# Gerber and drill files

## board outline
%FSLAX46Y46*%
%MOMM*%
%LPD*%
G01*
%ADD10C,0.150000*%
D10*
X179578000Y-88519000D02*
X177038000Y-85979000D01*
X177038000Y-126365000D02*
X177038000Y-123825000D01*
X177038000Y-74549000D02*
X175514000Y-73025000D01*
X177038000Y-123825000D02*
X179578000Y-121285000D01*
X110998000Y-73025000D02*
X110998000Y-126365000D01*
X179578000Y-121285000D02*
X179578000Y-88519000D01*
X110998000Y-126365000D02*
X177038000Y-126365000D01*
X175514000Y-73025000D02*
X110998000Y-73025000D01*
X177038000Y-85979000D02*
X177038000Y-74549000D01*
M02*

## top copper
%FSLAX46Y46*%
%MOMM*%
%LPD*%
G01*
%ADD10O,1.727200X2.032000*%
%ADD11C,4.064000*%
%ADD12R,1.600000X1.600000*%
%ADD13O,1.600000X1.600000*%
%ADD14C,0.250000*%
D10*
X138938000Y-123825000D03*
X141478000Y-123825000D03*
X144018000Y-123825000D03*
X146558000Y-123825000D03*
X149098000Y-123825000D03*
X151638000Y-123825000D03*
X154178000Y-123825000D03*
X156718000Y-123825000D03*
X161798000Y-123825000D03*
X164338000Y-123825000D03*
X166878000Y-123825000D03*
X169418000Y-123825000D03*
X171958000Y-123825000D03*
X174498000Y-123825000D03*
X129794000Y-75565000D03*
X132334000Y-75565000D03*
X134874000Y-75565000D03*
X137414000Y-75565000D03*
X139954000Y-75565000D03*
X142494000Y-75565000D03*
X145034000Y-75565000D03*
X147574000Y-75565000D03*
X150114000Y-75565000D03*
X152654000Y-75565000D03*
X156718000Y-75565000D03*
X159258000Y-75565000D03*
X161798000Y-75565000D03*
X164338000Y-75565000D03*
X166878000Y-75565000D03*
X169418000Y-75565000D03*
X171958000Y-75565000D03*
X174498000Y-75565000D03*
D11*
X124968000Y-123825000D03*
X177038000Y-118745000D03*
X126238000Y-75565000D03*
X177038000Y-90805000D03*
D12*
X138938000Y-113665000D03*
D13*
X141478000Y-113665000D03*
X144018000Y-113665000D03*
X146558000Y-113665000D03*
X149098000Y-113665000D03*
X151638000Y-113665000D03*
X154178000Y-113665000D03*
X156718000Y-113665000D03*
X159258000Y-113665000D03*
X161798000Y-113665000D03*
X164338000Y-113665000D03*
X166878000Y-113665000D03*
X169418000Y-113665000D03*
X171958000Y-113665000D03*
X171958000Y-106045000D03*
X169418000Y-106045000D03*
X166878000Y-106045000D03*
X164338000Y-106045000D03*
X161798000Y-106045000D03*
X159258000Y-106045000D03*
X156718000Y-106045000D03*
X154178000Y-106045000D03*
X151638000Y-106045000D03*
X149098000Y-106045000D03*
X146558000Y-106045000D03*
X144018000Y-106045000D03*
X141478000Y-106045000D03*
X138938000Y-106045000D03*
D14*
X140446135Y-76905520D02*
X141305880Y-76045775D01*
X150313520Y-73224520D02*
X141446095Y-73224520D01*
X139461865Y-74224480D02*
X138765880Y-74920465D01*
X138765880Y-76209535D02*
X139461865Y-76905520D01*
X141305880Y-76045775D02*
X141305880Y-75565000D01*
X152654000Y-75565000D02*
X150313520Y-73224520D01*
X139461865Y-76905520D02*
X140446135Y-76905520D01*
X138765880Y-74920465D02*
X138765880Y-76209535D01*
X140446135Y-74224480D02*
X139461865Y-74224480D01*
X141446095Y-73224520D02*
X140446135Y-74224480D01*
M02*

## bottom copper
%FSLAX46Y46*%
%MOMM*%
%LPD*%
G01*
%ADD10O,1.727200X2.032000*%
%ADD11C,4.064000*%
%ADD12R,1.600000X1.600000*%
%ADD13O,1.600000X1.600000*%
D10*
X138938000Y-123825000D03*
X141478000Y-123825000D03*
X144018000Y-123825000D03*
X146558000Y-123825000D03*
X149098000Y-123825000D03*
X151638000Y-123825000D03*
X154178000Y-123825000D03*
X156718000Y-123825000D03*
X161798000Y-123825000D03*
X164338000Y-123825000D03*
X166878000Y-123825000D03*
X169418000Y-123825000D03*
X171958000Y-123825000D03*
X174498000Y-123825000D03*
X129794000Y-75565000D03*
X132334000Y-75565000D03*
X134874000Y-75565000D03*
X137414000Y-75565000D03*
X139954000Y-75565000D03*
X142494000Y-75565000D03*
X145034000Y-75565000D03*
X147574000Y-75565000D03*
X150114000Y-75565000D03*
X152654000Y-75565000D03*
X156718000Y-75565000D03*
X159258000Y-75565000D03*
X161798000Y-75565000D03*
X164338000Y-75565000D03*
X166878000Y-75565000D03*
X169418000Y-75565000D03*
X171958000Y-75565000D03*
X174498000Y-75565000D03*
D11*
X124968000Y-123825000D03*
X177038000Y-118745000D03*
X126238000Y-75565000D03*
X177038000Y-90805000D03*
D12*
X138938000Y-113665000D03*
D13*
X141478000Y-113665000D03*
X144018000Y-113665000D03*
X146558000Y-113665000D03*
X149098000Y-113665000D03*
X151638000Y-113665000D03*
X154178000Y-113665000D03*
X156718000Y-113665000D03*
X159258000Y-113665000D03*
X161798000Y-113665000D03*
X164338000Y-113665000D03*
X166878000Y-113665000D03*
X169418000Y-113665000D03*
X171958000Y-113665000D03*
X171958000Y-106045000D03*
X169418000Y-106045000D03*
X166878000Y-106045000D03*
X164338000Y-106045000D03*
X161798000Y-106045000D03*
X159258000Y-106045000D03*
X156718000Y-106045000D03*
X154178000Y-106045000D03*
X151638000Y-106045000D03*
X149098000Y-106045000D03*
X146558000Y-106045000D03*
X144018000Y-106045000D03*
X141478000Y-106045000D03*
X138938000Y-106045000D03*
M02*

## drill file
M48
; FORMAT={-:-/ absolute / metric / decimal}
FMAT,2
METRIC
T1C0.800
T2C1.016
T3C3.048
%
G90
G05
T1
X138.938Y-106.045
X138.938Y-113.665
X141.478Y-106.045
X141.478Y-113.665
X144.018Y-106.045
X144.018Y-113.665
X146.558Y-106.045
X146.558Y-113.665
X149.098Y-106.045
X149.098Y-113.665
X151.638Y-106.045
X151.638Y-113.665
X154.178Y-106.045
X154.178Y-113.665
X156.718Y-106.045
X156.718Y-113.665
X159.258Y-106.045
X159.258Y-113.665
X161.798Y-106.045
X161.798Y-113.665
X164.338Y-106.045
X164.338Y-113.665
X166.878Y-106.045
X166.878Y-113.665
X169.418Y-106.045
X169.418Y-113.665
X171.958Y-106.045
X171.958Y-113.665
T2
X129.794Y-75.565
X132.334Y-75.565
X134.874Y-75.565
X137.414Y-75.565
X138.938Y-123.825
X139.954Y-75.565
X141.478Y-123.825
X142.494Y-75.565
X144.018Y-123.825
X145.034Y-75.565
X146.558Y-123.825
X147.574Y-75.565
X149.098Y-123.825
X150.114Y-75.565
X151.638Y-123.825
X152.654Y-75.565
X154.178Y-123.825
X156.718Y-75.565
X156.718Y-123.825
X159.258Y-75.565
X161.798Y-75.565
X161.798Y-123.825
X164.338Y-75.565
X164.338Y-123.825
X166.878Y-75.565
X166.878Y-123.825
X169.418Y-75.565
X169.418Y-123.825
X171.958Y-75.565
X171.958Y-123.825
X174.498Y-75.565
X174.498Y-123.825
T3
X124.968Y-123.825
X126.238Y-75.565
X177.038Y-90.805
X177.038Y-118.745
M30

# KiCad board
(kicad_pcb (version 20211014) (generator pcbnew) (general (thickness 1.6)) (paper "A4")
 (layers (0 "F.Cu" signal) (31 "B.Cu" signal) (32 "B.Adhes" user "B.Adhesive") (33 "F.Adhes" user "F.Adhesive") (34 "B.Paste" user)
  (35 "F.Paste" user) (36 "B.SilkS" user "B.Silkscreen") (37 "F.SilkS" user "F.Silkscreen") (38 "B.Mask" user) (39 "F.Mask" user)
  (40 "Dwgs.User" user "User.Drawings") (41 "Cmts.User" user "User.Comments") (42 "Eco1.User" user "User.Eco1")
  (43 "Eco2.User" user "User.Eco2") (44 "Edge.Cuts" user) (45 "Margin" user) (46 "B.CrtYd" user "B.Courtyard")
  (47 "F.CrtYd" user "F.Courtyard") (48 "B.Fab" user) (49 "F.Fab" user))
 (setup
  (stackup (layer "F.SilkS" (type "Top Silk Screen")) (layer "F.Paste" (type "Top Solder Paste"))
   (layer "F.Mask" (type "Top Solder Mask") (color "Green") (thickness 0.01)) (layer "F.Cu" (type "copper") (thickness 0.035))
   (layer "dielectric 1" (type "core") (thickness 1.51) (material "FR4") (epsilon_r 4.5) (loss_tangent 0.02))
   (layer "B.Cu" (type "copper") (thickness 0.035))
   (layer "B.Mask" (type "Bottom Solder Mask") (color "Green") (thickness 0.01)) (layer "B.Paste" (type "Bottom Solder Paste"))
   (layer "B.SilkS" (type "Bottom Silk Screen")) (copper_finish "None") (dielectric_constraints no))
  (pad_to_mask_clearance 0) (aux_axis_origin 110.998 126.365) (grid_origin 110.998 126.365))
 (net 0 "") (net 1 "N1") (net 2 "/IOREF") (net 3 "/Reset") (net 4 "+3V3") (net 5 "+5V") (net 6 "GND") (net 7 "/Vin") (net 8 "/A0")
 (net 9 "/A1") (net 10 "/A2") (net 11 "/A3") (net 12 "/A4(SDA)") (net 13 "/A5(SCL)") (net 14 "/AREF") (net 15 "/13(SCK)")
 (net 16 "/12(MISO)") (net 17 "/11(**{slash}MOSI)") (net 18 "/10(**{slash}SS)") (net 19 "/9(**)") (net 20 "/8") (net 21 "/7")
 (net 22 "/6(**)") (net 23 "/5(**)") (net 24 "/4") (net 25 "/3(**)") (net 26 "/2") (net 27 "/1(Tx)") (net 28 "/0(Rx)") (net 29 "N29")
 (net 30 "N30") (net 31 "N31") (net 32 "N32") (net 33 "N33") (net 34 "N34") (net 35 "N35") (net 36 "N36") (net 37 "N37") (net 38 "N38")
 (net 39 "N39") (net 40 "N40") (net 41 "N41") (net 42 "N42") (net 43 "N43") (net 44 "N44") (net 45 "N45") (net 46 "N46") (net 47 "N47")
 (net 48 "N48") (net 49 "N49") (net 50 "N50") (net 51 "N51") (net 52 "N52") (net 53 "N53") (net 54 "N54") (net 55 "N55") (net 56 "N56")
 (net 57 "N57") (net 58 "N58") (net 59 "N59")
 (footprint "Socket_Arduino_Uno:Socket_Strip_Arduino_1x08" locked (layer "F.Cu") (at 138.938 123.825)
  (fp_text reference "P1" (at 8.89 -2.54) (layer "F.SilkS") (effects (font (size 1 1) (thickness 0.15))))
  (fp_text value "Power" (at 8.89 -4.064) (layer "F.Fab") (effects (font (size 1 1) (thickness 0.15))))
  (pad "1" thru_hole oval locked (at 0 0) (size 1.7272 2.032) (drill 1.016) (layers *.Cu *.Mask "F.SilkS") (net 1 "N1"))
  (pad "2" thru_hole oval locked (at 2.54 0) (size 1.7272 2.032) (drill 1.016) (layers *.Cu *.Mask "F.SilkS") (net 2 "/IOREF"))
  (pad "3" thru_hole oval locked (at 5.08 0) (size 1.7272 2.032) (drill 1.016) (layers *.Cu *.Mask "F.SilkS") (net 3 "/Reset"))
  (pad "4" thru_hole oval locked (at 7.62 0) (size 1.7272 2.032) (drill 1.016) (layers *.Cu *.Mask "F.SilkS") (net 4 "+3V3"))
  (pad "5" thru_hole oval locked (at 10.16 0) (size 1.7272 2.032) (drill 1.016) (layers *.Cu *.Mask "F.SilkS") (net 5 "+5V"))
  (pad "6" thru_hole oval locked (at 12.7 0) (size 1.7272 2.032) (drill 1.016) (layers *.Cu *.Mask "F.SilkS") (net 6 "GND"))
  (pad "7" thru_hole oval locked (at 15.24 0) (size 1.7272 2.032) (drill 1.016) (layers *.Cu *.Mask "F.SilkS") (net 6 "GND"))
  (pad "8" thru_hole oval locked (at 17.78 0) (size 1.7272 2.032) (drill 1.016) (layers *.Cu *.Mask "F.SilkS") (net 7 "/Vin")))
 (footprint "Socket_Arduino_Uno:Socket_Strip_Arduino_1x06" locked (layer "F.Cu") (at 161.798 123.825)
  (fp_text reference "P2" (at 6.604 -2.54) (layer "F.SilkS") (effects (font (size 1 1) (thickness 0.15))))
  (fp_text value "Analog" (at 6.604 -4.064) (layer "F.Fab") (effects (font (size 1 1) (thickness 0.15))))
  (pad "1" thru_hole oval locked (at 0 0) (size 1.7272 2.032) (drill 1.016) (layers *.Cu *.Mask "F.SilkS") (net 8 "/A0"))
  (pad "2" thru_hole oval locked (at 2.54 0) (size 1.7272 2.032) (drill 1.016) (layers *.Cu *.Mask "F.SilkS") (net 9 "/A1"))
  (pad "3" thru_hole oval locked (at 5.08 0) (size 1.7272 2.032) (drill 1.016) (layers *.Cu *.Mask "F.SilkS") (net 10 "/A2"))
  (pad "4" thru_hole oval locked (at 7.62 0) (size 1.7272 2.032) (drill 1.016) (layers *.Cu *.Mask "F.SilkS") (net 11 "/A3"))
  (pad "5" thru_hole oval locked (at 10.16 0) (size 1.7272 2.032) (drill 1.016) (layers *.Cu *.Mask "F.SilkS") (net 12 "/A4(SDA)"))
  (pad "6" thru_hole oval locked (at 12.7 0) (size 1.7272 2.032) (drill 1.016) (layers *.Cu *.Mask "F.SilkS") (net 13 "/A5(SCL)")))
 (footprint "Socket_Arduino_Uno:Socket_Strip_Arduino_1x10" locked (layer "F.Cu") (at 129.794 75.565)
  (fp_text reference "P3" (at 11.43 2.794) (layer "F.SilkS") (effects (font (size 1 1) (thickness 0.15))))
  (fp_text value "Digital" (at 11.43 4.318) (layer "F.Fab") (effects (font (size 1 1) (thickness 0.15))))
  (pad "1" thru_hole oval locked (at 0 0) (size 1.7272 2.032) (drill 1.016) (layers *.Cu *.Mask "F.SilkS") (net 13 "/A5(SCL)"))
  (pad "2" thru_hole oval locked (at 2.54 0) (size 1.7272 2.032) (drill 1.016) (layers *.Cu *.Mask "F.SilkS") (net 12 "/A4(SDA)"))
  (pad "3" thru_hole oval locked (at 5.08 0) (size 1.7272 2.032) (drill 1.016) (layers *.Cu *.Mask "F.SilkS") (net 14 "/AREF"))
  (pad "4" thru_hole oval locked (at 7.62 0) (size 1.7272 2.032) (drill 1.016) (layers *.Cu *.Mask "F.SilkS") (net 6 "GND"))
  (pad "5" thru_hole oval locked (at 10.16 0) (size 1.7272 2.032) (drill 1.016) (layers *.Cu *.Mask "F.SilkS") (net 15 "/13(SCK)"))
  (pad "6" thru_hole oval locked (at 12.7 0) (size 1.7272 2.032) (drill 1.016) (layers *.Cu *.Mask "F.SilkS") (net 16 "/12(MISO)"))
  (pad "7" thru_hole oval locked (at 15.24 0) (size 1.7272 2.032) (drill 1.016) (layers *.Cu *.Mask "F.SilkS") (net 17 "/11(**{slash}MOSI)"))
  (pad "8" thru_hole oval locked (at 17.78 0) (size 1.7272 2.032) (drill 1.016) (layers *.Cu *.Mask "F.SilkS") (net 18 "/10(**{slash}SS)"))
  (pad "9" thru_hole oval locked (at 20.32 0) (size 1.7272 2.032) (drill 1.016) (layers *.Cu *.Mask "F.SilkS") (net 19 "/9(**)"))
  (pad "10" thru_hole oval locked (at 22.86 0) (size 1.7272 2.032) (drill 1.016) (layers *.Cu *.Mask "F.SilkS") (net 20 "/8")))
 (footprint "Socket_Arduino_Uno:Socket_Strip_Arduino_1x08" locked (layer "F.Cu") (at 156.718 75.565)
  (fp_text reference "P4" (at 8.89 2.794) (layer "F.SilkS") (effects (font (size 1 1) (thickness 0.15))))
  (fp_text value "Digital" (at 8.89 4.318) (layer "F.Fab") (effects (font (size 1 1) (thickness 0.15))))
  (pad "1" thru_hole oval locked (at 0 0) (size 1.7272 2.032) (drill 1.016) (layers *.Cu *.Mask "F.SilkS") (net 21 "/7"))
  (pad "2" thru_hole oval locked (at 2.54 0) (size 1.7272 2.032) (drill 1.016) (layers *.Cu *.Mask "F.SilkS") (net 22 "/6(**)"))
  (pad "3" thru_hole oval locked (at 5.08 0) (size 1.7272 2.032) (drill 1.016) (layers *.Cu *.Mask "F.SilkS") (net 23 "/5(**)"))
  (pad "4" thru_hole oval locked (at 7.62 0) (size 1.7272 2.032) (drill 1.016) (layers *.Cu *.Mask "F.SilkS") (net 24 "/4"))
  (pad "5" thru_hole oval locked (at 10.16 0) (size 1.7272 2.032) (drill 1.016) (layers *.Cu *.Mask "F.SilkS") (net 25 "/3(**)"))
  (pad "6" thru_hole oval locked (at 12.7 0) (size 1.7272 2.032) (drill 1.016) (layers *.Cu *.Mask "F.SilkS") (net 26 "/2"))
  (pad "7" thru_hole oval locked (at 15.24 0) (size 1.7272 2.032) (drill 1.016) (layers *.Cu *.Mask "F.SilkS") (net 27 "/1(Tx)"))
  (pad "8" thru_hole oval locked (at 17.78 0) (size 1.7272 2.032) (drill 1.016) (layers *.Cu *.Mask "F.SilkS") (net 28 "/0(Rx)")))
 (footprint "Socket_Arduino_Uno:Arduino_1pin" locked (layer "F.Cu") (at 124.968 123.825)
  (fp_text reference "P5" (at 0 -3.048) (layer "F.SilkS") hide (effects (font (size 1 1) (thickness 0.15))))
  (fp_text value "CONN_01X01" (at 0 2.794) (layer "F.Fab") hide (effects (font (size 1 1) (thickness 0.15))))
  (pad "1" thru_hole circle locked (at 0 0) (size 4.064 4.064) (drill 3.048) (layers *.Cu *.Mask "F.SilkS") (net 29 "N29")))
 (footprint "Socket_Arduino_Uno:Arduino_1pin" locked (layer "F.Cu") (at 177.038 118.745)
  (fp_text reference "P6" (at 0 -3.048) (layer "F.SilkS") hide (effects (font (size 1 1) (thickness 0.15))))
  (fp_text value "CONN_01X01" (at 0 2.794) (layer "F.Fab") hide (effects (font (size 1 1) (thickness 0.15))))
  (pad "1" thru_hole circle locked (at 0 0) (size 4.064 4.064) (drill 3.048) (layers *.Cu *.Mask "F.SilkS") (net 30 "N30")))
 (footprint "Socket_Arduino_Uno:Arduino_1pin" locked (layer "F.Cu") (at 126.238 75.565)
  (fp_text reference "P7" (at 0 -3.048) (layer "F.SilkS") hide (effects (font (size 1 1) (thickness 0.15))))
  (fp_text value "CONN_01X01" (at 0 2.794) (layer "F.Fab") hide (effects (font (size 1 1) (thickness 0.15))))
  (pad "1" thru_hole circle locked (at 0 0) (size 4.064 4.064) (drill 3.048) (layers *.Cu *.Mask "F.SilkS") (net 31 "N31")))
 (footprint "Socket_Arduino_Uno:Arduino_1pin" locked (layer "F.Cu") (at 177.038 90.805)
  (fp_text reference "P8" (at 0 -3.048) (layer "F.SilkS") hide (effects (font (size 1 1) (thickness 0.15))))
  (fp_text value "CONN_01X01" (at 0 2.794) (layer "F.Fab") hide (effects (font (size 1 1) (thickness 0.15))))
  (pad "1" thru_hole circle locked (at 0 0) (size 4.064 4.064) (drill 3.048) (layers *.Cu *.Mask "F.SilkS") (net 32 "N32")))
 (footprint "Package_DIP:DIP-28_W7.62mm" (layer "F.Cu") (at 138.938 113.665 90)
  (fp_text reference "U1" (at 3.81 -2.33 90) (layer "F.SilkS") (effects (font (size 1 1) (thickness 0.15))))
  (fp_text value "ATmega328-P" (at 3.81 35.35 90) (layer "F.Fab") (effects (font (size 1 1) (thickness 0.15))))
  (pad "1" thru_hole rect (at 0 0 90) (size 1.6 1.6) (drill 0.8) (layers *.Cu *.Mask) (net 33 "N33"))
  (pad "2" thru_hole oval (at 0 2.54 90) (size 1.6 1.6) (drill 0.8) (layers *.Cu *.Mask) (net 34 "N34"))
  (pad "3" thru_hole oval (at 0 5.08 90) (size 1.6 1.6) (drill 0.8) (layers *.Cu *.Mask) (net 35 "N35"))
  (pad "4" thru_hole oval (at 0 7.62 90) (size 1.6 1.6) (drill 0.8) (layers *.Cu *.Mask) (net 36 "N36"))
  (pad "5" thru_hole oval (at 0 10.16 90) (size 1.6 1.6) (drill 0.8) (layers *.Cu *.Mask) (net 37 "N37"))
  (pad "6" thru_hole oval (at 0 12.7 90) (size 1.6 1.6) (drill 0.8) (layers *.Cu *.Mask) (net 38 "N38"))
  (pad "7" thru_hole oval (at 0 15.24 90) (size 1.6 1.6) (drill 0.8) (layers *.Cu *.Mask) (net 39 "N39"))
  (pad "8" thru_hole oval (at 0 17.78 90) (size 1.6 1.6) (drill 0.8) (layers *.Cu *.Mask) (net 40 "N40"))
  (pad "9" thru_hole oval (at 0 20.32 90) (size 1.6 1.6) (drill 0.8) (layers *.Cu *.Mask) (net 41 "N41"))
  (pad "10" thru_hole oval (at 0 22.86 90) (size 1.6 1.6) (drill 0.8) (layers *.Cu *.Mask) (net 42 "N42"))
  (pad "11" thru_hole oval (at 0 25.4 90) (size 1.6 1.6) (drill 0.8) (layers *.Cu *.Mask) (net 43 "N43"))
  (pad "12" thru_hole oval (at 0 27.94 90) (size 1.6 1.6) (drill 0.8) (layers *.Cu *.Mask) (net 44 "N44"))
  (pad "13" thru_hole oval (at 0 30.48 90) (size 1.6 1.6) (drill 0.8) (layers *.Cu *.Mask) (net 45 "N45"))
  (pad "14" thru_hole oval (at 0 33.02 90) (size 1.6 1.6) (drill 0.8) (layers *.Cu *.Mask) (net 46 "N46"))
  (pad "15" thru_hole oval (at 7.62 33.02 90) (size 1.6 1.6) (drill 0.8) (layers *.Cu *.Mask) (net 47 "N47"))
  (pad "16" thru_hole oval (at 7.62 30.48 90) (size 1.6 1.6) (drill 0.8) (layers *.Cu *.Mask) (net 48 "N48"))
  (pad "17" thru_hole oval (at 7.62 27.94 90) (size 1.6 1.6) (drill 0.8) (layers *.Cu *.Mask) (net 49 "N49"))
  (pad "18" thru_hole oval (at 7.62 25.4 90) (size 1.6 1.6) (drill 0.8) (layers *.Cu *.Mask) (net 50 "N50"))
  (pad "19" thru_hole oval (at 7.62 22.86 90) (size 1.6 1.6) (drill 0.8) (layers *.Cu *.Mask) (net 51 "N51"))
  (pad "20" thru_hole oval (at 7.62 20.32 90) (size 1.6 1.6) (drill 0.8) (layers *.Cu *.Mask) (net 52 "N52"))
  (pad "21" thru_hole oval (at 7.62 17.78 90) (size 1.6 1.6) (drill 0.8) (layers *.Cu *.Mask) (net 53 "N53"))
  (pad "22" thru_hole oval (at 7.62 15.24 90) (size 1.6 1.6) (drill 0.8) (layers *.Cu *.Mask) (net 40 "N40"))
  (pad "23" thru_hole oval (at 7.62 12.7 90) (size 1.6 1.6) (drill 0.8) (layers *.Cu *.Mask) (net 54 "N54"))
  (pad "24" thru_hole oval (at 7.62 10.16 90) (size 1.6 1.6) (drill 0.8) (layers *.Cu *.Mask) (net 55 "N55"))
  (pad "25" thru_hole oval (at 7.62 7.62 90) (size 1.6 1.6) (drill 0.8) (layers *.Cu *.Mask) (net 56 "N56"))
  (pad "26" thru_hole oval (at 7.62 5.08 90) (size 1.6 1.6) (drill 0.8) (layers *.Cu *.Mask) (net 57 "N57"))
  (pad "27" thru_hole oval (at 7.62 2.54 90) (size 1.6 1.6) (drill 0.8) (layers *.Cu *.Mask) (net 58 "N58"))
  (pad "28" thru_hole oval (at 7.62 0 90) (size 1.6 1.6) (drill 0.8) (layers *.Cu *.Mask) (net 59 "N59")))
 (gr_line (start 179.578 88.519) (end 177.038 85.979) (layer "Edge.Cuts") (width 0.15))
 (gr_line (start 177.038 126.365) (end 177.038 123.825) (layer "Edge.Cuts") (width 0.15))
 (gr_line (start 177.038 74.549) (end 175.514 73.025) (layer "Edge.Cuts") (width 0.15))
 (gr_line (start 177.038 123.825) (end 179.578 121.285) (layer "Edge.Cuts") (width 0.15))
 (gr_line (start 110.998 73.025) (end 110.998 126.365) (layer "Edge.Cuts") (width 0.15))
 (gr_line (start 179.578 121.285) (end 179.578 88.519) (layer "Edge.Cuts") (width 0.15))
 (gr_line (start 110.998 126.365) (end 177.038 126.365) (layer "Edge.Cuts") (width 0.15))
 (gr_line (start 175.514 73.025) (end 110.998 73.025) (layer "Edge.Cuts") (width 0.15))
 (gr_line (start 177.038 85.979) (end 177.038 74.549) (layer "Edge.Cuts") (width 0.15))
 (segment (start 140.446135 76.90552) (end 141.30588 76.045775) (width 0.25) (layer "F.Cu") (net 20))
 (segment (start 150.31352 73.22452) (end 141.446095 73.22452) (width 0.25) (layer "F.Cu") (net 20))
 (segment (start 139.461865 74.22448) (end 138.76588 74.920465) (width 0.25) (layer "F.Cu") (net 20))
 (segment (start 138.76588 76.209535) (end 139.461865 76.90552) (width 0.25) (layer "F.Cu") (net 20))
 (segment (start 141.30588 76.045775) (end 141.30588 75.565) (width 0.25) (layer "F.Cu") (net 20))
 (segment (start 152.654 75.565) (end 150.31352 73.22452) (width 0.25) (layer "F.Cu") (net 20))
 (segment (start 139.461865 76.90552) (end 140.446135 76.90552) (width 0.25) (layer "F.Cu") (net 20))
 (segment (start 138.76588 74.920465) (end 138.76588 76.209535) (width 0.25) (layer "F.Cu") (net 20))
 (segment (start 140.446135 74.22448) (end 139.461865 74.22448) (width 0.25) (layer "F.Cu") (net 20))
 (segment (start 141.446095 73.22452) (end 140.446135 74.22448) (width 0.25) (layer "F.Cu") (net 20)))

